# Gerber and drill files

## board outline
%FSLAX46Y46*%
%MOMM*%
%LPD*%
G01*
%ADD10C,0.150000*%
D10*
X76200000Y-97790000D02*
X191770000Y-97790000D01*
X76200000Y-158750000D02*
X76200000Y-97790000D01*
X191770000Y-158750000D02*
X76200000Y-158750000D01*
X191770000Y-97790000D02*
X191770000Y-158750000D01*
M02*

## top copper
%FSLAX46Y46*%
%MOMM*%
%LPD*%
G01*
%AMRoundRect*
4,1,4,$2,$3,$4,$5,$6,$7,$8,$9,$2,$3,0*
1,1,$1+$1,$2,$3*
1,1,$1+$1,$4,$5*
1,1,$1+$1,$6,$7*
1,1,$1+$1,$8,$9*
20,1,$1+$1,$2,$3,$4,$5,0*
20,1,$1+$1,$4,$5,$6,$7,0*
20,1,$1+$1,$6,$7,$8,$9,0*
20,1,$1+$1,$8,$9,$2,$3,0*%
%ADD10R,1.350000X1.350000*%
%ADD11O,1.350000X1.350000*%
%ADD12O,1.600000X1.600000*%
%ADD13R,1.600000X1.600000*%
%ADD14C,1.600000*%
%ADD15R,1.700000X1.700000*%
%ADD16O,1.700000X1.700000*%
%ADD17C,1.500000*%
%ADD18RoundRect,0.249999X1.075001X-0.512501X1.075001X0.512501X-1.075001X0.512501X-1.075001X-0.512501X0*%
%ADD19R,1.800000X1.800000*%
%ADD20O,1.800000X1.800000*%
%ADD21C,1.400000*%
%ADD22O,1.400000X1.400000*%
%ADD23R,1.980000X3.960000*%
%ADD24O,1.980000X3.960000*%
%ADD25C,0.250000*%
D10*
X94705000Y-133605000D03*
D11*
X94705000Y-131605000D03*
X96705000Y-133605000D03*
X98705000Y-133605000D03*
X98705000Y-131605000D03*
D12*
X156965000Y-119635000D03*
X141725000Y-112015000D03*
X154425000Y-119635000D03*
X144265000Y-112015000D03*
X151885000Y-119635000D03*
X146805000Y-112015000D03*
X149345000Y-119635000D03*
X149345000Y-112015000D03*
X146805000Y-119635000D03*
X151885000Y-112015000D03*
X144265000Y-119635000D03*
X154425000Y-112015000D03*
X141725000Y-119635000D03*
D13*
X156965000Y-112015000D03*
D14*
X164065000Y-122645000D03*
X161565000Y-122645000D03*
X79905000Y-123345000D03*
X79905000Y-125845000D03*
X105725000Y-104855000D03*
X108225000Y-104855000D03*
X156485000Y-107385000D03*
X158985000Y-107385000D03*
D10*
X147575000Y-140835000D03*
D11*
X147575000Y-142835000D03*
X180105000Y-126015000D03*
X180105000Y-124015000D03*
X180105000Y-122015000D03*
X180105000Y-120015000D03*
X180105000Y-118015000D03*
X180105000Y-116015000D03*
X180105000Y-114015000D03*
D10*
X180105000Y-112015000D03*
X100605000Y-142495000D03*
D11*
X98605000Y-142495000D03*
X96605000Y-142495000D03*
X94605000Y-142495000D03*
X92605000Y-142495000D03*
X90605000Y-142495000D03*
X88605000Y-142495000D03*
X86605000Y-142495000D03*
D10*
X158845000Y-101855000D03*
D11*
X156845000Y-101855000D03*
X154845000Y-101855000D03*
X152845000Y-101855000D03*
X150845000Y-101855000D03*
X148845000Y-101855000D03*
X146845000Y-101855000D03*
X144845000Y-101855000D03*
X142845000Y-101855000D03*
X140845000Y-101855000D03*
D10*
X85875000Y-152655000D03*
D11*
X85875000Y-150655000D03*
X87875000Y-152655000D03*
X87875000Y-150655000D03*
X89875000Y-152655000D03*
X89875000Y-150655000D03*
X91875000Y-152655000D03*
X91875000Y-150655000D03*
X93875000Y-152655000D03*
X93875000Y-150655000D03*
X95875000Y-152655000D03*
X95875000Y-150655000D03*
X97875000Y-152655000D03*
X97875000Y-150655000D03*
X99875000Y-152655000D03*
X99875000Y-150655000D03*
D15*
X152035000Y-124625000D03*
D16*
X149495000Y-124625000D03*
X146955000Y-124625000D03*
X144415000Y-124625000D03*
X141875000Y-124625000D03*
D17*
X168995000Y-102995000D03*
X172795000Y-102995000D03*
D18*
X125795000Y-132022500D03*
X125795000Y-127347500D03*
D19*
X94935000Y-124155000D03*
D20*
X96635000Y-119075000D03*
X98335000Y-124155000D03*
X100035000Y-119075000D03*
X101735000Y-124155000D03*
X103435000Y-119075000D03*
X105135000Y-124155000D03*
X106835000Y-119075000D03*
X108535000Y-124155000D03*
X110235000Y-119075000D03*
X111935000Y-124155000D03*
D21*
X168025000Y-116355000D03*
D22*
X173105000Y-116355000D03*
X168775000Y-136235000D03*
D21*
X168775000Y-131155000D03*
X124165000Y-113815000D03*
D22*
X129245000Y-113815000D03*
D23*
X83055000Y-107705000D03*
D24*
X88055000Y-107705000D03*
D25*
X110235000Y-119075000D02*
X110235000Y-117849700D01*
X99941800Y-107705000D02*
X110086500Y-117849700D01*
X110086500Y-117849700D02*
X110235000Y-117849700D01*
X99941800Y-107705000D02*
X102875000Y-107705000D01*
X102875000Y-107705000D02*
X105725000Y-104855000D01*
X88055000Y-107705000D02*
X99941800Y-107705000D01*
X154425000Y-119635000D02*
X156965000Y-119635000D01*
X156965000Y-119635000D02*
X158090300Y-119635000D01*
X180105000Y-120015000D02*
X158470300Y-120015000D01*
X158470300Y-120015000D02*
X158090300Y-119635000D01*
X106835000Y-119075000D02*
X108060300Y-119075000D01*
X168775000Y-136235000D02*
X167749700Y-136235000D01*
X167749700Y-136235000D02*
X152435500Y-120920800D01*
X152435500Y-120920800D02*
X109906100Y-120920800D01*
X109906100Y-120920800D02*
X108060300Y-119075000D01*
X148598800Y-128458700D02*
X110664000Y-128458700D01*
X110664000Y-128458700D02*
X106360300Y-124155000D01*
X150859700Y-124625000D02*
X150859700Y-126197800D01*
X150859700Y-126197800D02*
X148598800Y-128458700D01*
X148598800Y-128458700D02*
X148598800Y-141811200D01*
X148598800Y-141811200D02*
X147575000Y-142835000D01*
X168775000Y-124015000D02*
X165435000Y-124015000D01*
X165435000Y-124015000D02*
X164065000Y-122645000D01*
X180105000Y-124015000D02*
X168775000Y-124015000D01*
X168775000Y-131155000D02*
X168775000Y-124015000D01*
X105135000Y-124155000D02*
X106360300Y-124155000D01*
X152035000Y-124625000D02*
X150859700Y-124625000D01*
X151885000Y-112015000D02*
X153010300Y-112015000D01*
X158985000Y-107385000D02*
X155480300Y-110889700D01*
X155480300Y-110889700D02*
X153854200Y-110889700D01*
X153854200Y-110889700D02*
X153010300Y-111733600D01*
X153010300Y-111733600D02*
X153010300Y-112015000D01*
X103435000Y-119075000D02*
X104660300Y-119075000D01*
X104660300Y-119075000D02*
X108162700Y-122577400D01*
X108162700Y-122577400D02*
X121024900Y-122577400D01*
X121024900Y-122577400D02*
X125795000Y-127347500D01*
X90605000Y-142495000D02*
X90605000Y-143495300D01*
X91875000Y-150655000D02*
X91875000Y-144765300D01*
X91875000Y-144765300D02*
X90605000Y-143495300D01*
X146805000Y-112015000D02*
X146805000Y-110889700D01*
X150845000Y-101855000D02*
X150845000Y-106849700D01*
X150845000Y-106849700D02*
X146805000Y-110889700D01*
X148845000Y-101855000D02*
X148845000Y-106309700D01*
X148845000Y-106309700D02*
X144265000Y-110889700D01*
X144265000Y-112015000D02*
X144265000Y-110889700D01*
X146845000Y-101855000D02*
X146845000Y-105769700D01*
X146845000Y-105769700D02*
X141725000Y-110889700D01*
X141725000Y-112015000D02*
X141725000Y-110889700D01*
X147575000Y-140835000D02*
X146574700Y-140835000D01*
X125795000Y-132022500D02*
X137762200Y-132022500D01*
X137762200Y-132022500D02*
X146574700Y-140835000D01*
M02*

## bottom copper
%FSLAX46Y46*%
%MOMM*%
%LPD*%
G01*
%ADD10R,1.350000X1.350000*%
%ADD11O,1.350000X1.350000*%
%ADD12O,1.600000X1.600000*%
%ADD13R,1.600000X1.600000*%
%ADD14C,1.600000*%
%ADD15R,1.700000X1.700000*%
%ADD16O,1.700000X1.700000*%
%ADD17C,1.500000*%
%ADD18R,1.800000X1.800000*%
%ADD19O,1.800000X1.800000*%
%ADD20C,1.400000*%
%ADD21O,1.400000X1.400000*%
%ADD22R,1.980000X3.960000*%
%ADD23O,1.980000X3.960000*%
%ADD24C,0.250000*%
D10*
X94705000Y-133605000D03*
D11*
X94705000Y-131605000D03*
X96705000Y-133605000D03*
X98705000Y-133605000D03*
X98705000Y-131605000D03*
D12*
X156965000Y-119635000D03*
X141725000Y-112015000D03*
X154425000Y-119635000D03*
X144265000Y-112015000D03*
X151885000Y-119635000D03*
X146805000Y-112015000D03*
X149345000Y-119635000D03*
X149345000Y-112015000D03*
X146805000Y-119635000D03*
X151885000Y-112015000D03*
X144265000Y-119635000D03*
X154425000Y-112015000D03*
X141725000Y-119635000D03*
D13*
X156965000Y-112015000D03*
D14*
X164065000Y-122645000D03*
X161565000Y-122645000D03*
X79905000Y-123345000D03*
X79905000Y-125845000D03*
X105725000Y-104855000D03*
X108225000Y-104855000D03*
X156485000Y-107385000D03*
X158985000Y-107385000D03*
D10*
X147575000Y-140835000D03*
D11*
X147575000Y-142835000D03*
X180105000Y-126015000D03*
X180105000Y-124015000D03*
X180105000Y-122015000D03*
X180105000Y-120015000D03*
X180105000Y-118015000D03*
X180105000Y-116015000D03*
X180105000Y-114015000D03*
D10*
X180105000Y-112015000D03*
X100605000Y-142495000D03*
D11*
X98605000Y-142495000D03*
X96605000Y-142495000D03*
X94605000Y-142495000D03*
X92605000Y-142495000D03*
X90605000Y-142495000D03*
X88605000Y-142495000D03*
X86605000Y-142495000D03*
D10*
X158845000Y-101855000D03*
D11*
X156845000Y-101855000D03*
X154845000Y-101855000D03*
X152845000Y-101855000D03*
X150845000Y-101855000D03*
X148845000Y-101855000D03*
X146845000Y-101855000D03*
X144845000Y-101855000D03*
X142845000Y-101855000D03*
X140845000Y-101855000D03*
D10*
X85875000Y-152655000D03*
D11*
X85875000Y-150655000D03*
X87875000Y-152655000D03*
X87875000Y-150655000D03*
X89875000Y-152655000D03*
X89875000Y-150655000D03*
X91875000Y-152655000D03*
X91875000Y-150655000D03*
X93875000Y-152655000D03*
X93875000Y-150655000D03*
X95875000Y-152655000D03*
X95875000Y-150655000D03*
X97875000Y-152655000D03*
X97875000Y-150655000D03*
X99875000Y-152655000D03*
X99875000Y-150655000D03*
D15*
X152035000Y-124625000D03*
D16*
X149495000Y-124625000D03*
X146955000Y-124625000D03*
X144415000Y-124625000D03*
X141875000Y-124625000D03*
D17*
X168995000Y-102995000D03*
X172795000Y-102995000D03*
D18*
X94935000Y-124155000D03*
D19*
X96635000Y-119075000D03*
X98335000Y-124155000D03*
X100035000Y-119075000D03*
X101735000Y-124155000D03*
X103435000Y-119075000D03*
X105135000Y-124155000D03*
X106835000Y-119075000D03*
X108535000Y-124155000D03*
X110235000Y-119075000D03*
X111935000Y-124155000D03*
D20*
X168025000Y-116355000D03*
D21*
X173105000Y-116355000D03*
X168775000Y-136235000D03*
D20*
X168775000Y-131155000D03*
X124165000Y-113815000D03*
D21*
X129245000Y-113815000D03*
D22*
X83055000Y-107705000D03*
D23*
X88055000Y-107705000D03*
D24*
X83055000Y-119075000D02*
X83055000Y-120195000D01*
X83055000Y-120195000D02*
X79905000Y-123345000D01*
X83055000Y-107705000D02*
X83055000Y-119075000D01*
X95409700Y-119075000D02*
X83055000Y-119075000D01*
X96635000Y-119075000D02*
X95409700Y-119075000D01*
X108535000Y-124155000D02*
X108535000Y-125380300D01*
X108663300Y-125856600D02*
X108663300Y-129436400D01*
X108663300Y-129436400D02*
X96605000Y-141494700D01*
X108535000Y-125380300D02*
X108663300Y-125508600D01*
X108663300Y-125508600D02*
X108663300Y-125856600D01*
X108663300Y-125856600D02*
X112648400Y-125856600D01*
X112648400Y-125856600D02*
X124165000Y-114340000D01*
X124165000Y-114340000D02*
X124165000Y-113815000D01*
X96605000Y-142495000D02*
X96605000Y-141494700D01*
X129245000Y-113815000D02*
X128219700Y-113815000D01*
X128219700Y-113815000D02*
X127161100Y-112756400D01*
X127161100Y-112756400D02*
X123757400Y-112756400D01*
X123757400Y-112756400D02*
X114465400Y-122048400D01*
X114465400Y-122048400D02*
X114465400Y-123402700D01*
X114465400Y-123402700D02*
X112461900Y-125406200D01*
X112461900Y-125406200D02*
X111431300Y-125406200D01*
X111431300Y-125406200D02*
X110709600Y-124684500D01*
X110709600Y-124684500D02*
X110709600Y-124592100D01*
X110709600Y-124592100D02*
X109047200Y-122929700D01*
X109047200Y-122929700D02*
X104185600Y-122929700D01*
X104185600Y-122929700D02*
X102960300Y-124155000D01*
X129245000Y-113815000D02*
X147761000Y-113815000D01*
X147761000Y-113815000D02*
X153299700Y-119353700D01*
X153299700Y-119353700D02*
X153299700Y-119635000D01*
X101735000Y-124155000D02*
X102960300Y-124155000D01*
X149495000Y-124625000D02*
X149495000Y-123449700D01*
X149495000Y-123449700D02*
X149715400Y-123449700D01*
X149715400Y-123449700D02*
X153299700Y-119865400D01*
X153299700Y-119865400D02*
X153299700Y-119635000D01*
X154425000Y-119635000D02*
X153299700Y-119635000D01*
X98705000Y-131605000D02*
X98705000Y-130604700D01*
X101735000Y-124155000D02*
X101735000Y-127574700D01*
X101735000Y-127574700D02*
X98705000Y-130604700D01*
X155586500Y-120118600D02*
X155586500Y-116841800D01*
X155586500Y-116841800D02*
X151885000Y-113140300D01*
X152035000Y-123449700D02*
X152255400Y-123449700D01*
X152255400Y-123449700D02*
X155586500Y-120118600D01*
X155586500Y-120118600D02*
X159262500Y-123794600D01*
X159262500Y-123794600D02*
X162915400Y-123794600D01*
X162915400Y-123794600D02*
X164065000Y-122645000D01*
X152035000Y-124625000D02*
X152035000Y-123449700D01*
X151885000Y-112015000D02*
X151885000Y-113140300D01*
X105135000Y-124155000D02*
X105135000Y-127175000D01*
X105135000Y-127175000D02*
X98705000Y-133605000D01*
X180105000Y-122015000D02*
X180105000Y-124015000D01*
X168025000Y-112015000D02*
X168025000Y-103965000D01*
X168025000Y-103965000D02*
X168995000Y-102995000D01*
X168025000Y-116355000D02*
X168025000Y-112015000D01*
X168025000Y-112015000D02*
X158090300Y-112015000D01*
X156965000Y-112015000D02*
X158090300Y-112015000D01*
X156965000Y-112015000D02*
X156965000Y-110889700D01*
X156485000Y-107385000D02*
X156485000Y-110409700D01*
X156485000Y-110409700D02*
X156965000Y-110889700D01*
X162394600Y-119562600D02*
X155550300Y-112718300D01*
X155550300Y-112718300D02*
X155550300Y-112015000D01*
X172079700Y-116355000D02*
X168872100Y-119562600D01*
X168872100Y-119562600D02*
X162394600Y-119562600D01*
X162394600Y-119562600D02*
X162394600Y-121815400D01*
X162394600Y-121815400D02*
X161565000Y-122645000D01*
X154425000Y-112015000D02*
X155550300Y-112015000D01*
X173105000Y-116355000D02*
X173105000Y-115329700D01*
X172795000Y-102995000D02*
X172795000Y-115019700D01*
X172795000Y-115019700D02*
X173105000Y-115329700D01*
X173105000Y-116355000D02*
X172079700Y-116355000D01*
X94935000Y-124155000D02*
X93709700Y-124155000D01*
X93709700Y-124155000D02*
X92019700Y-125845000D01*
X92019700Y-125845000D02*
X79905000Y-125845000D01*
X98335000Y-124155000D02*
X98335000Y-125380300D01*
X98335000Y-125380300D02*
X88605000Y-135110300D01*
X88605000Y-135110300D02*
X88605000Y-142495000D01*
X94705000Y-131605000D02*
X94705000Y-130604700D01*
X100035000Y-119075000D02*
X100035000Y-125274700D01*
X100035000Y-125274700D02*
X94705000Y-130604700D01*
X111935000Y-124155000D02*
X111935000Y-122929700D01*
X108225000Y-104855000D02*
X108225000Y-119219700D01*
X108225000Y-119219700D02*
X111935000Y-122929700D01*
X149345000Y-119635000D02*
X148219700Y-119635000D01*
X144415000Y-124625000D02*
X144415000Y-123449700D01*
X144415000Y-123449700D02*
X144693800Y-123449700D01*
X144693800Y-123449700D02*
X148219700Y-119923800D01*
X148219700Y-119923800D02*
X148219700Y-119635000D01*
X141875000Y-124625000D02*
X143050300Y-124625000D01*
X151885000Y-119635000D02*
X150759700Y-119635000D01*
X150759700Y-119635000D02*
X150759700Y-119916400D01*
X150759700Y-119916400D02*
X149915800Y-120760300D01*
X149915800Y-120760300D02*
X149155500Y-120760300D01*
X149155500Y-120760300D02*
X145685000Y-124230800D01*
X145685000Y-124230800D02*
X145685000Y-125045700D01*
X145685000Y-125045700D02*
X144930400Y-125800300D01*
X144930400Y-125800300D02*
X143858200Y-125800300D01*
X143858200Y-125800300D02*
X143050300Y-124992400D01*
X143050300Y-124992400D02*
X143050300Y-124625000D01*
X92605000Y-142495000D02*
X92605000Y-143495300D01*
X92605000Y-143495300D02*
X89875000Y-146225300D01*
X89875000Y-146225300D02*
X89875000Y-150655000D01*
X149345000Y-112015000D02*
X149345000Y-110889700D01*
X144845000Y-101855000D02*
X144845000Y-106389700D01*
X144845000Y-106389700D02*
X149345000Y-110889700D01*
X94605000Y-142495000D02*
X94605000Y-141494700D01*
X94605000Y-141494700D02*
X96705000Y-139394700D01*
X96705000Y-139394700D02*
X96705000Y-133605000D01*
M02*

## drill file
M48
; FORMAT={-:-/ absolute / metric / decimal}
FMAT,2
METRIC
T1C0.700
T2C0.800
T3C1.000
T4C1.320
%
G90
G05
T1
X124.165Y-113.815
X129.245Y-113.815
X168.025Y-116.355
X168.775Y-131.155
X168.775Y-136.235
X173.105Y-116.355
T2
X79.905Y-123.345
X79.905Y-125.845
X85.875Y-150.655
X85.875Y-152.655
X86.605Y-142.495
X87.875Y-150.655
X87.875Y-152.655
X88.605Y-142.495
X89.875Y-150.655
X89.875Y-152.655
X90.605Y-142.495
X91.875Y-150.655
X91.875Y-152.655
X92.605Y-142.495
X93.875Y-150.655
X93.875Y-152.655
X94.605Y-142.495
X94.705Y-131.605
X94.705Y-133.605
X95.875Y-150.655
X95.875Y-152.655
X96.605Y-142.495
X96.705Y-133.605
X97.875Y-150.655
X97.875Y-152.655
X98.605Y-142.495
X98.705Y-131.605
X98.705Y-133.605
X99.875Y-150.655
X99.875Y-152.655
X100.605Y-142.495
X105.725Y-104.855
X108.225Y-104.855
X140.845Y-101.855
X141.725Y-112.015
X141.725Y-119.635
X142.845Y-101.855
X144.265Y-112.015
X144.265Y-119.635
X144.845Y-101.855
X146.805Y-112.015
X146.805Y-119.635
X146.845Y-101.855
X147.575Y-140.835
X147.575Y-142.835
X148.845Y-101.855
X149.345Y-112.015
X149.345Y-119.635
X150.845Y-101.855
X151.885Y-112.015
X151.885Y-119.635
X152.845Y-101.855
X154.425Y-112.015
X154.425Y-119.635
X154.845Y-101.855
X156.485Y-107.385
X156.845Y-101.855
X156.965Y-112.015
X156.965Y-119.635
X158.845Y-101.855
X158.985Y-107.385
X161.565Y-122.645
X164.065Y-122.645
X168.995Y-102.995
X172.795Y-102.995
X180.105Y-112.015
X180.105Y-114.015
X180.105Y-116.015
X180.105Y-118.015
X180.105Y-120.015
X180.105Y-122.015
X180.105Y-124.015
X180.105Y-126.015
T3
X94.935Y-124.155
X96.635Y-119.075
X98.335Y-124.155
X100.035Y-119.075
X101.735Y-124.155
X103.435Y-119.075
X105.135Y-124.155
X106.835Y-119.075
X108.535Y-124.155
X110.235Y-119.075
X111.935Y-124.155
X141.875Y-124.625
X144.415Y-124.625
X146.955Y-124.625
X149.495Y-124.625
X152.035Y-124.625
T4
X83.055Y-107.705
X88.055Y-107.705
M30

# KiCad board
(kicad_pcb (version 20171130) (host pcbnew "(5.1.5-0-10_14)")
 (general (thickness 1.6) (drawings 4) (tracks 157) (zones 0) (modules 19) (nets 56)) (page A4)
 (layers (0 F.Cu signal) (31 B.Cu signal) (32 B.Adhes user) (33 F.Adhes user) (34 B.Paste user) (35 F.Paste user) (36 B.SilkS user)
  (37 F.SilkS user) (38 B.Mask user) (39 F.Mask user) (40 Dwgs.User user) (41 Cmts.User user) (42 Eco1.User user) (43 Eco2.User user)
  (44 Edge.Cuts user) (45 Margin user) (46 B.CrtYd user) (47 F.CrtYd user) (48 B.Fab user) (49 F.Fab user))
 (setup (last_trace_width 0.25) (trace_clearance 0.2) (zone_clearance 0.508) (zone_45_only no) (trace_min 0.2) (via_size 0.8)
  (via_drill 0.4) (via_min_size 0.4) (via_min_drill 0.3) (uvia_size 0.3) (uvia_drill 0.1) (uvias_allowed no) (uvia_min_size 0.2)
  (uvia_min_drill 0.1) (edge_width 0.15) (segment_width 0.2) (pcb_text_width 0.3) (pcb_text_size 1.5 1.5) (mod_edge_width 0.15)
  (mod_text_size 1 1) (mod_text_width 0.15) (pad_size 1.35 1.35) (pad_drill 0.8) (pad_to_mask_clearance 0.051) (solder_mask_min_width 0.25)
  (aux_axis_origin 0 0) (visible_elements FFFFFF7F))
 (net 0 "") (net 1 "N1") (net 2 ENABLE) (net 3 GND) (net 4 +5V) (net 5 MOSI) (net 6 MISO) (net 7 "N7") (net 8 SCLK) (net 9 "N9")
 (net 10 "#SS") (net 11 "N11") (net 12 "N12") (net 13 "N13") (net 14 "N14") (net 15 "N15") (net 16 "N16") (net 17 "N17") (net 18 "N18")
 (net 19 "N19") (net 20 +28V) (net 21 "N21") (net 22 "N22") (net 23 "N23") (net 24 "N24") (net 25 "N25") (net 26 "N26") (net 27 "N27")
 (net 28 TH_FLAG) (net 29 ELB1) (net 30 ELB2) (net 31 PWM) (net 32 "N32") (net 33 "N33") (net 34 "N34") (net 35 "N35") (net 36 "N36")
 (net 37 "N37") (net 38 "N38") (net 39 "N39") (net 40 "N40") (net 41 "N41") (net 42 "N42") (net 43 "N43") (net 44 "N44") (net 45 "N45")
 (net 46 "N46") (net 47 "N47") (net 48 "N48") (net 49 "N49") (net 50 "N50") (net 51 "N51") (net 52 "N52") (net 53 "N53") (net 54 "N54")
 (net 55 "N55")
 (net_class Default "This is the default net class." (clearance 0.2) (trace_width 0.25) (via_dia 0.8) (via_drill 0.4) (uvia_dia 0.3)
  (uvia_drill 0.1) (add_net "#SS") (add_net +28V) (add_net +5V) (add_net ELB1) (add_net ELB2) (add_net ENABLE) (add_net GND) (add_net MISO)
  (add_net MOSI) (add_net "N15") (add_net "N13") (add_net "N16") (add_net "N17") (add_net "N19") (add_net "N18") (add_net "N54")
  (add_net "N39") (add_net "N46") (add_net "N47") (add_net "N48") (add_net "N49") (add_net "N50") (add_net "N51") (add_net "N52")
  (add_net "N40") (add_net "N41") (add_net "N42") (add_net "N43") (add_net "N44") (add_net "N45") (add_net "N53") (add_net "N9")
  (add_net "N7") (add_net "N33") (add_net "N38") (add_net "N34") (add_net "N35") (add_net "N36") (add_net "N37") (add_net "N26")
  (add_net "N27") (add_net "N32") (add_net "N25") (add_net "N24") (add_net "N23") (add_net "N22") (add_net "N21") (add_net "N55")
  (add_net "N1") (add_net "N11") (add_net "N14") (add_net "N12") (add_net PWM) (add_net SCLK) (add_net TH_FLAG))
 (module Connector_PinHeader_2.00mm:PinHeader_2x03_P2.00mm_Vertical (layer F.Cu) (at 94.705 133.605 90)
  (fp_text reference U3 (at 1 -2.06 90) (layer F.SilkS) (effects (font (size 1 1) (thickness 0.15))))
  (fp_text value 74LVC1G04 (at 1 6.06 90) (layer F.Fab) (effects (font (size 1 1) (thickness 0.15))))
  (pad 1 thru_hole rect (at 0 0 90) (size 1.35 1.35) (drill 0.8) (layers *.Cu *.Mask))
  (pad 4 thru_hole oval (at 2 0 90) (size 1.35 1.35) (drill 0.8) (layers *.Cu *.Mask) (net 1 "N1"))
  (pad 2 thru_hole oval (at 0 2 90) (size 1.35 1.35) (drill 0.8) (layers *.Cu *.Mask) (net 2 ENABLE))
  (pad 3 thru_hole oval (at 0 4 90) (size 1.35 1.35) (drill 0.8) (layers *.Cu *.Mask) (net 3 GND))
  (pad 5 thru_hole oval (at 2 4 90) (size 1.35 1.35) (drill 0.8) (layers *.Cu *.Mask) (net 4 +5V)))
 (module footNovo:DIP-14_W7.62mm (layer F.Cu) (at 156.965 112.015 270)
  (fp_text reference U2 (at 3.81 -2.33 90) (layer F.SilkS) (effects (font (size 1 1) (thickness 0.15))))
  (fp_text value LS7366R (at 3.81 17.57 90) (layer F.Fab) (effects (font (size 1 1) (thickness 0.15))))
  (pad 14 thru_hole oval (at 7.62 0 270) (size 1.6 1.6) (drill 0.8) (layers *.Cu *.Mask) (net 4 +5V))
  (pad 7 thru_hole oval (at 0 15.24 270) (size 1.6 1.6) (drill 0.8) (layers *.Cu *.Mask) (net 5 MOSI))
  (pad 13 thru_hole oval (at 7.62 2.54 270) (size 1.6 1.6) (drill 0.8) (layers *.Cu *.Mask) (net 4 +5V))
  (pad 6 thru_hole oval (at 0 12.7 270) (size 1.6 1.6) (drill 0.8) (layers *.Cu *.Mask) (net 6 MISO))
  (pad 12 thru_hole oval (at 7.62 5.08 270) (size 1.6 1.6) (drill 0.8) (layers *.Cu *.Mask) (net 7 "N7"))
  (pad 5 thru_hole oval (at 0 10.16 270) (size 1.6 1.6) (drill 0.8) (layers *.Cu *.Mask) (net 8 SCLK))
  (pad 11 thru_hole oval (at 7.62 7.62 270) (size 1.6 1.6) (drill 0.8) (layers *.Cu *.Mask) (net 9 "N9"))
  (pad 4 thru_hole oval (at 0 7.62 270) (size 1.6 1.6) (drill 0.8) (layers *.Cu *.Mask) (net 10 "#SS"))
  (pad 10 thru_hole oval (at 7.62 10.16 270) (size 1.6 1.6) (drill 0.8) (layers *.Cu *.Mask) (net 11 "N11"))
  (pad 3 thru_hole oval (at 0 5.08 270) (size 1.6 1.6) (drill 0.8) (layers *.Cu *.Mask) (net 3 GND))
  (pad 9 thru_hole oval (at 7.62 12.7 270) (size 1.6 1.6) (drill 0.8) (layers *.Cu *.Mask) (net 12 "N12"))
  (pad 2 thru_hole oval (at 0 2.54 270) (size 1.6 1.6) (drill 0.8) (layers *.Cu *.Mask) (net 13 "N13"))
  (pad 8 thru_hole oval (at 7.62 15.24 270) (size 1.6 1.6) (drill 0.8) (layers *.Cu *.Mask) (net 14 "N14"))
  (pad 1 thru_hole rect (at 0 0 270) (size 1.6 1.6) (drill 0.8) (layers *.Cu *.Mask) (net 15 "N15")))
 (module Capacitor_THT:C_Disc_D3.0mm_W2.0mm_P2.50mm (layer F.Cu) (at 161.565 122.645)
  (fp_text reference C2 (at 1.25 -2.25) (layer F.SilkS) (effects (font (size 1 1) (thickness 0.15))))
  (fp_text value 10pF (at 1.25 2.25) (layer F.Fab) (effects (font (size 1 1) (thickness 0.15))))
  (pad 2 thru_hole circle (at 2.5 0) (size 1.6 1.6) (drill 0.8) (layers *.Cu *.Mask) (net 3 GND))
  (pad 1 thru_hole circle (at 0 0) (size 1.6 1.6) (drill 0.8) (layers *.Cu *.Mask) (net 13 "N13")))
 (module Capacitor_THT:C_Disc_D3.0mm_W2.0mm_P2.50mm (layer F.Cu) (at 79.905 123.345 270)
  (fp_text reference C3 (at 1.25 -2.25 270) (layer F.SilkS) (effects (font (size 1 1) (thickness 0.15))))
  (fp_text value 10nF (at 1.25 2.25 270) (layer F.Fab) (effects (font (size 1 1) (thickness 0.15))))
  (pad 1 thru_hole circle (at 0 0 270) (size 1.6 1.6) (drill 0.8) (layers *.Cu *.Mask) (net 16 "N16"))
  (pad 2 thru_hole circle (at 2.5 0 270) (size 1.6 1.6) (drill 0.8) (layers *.Cu *.Mask) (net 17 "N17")))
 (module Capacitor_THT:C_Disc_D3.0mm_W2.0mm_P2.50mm (layer F.Cu) (at 108.225 104.855 180)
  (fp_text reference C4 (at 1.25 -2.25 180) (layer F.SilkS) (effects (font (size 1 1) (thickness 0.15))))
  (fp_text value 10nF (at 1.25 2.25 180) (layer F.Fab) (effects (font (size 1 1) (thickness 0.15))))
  (pad 2 thru_hole circle (at 2.5 0 180) (size 1.6 1.6) (drill 0.8) (layers *.Cu *.Mask) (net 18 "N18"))
  (pad 1 thru_hole circle (at 0 0 180) (size 1.6 1.6) (drill 0.8) (layers *.Cu *.Mask) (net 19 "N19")))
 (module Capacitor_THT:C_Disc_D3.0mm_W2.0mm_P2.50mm (layer F.Cu) (at 156.485 107.385)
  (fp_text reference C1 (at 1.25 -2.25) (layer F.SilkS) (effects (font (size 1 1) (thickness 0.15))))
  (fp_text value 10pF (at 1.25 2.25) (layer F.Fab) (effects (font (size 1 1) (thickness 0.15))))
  (pad 1 thru_hole circle (at 0 0) (size 1.6 1.6) (drill 0.8) (layers *.Cu *.Mask) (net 15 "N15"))
  (pad 2 thru_hole circle (at 2.5 0) (size 1.6 1.6) (drill 0.8) (layers *.Cu *.Mask) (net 3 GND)))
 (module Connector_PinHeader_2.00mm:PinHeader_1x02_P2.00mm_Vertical (layer F.Cu) (at 147.575 140.835)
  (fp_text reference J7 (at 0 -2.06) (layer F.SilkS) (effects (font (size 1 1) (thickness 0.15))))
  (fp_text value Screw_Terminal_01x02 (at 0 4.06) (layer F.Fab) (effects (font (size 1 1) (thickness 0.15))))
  (pad 1 thru_hole rect (at 0 0) (size 1.35 1.35) (drill 0.8) (layers *.Cu *.Mask) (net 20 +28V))
  (pad 2 thru_hole oval (at 0 2) (size 1.35 1.35) (drill 0.8) (layers *.Cu *.Mask) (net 3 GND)))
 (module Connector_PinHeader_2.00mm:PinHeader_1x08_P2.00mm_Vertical (layer F.Cu) (at 180.105 112.015)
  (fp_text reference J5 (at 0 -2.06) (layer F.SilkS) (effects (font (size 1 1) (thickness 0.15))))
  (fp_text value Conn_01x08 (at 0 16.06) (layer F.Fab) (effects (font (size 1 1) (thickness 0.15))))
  (pad 8 thru_hole oval (at 0 14) (size 1.35 1.35) (drill 0.8) (layers *.Cu *.Mask) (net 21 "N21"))
  (pad 7 thru_hole oval (at 0 12) (size 1.35 1.35) (drill 0.8) (layers *.Cu *.Mask) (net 3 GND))
  (pad 6 thru_hole oval (at 0 10) (size 1.35 1.35) (drill 0.8) (layers *.Cu *.Mask) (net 3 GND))
  (pad 5 thru_hole oval (at 0 8) (size 1.35 1.35) (drill 0.8) (layers *.Cu *.Mask) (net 4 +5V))
  (pad 4 thru_hole oval (at 0 6) (size 1.35 1.35) (drill 0.8) (layers *.Cu *.Mask) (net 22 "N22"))
  (pad 3 thru_hole oval (at 0 4) (size 1.35 1.35) (drill 0.8) (layers *.Cu *.Mask) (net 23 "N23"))
  (pad 2 thru_hole oval (at 0 2) (size 1.35 1.35) (drill 0.8) (layers *.Cu *.Mask) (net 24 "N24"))
  (pad 1 thru_hole rect (at 0 0) (size 1.35 1.35) (drill 0.8) (layers *.Cu *.Mask) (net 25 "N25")))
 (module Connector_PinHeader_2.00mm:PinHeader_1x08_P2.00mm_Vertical (layer F.Cu) (at 100.605 142.495 270)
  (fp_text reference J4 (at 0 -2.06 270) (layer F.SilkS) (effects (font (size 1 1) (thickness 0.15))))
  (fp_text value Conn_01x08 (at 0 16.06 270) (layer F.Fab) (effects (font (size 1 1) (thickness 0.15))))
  (pad 1 thru_hole rect (at 0 0 270) (size 1.35 1.35) (drill 0.8) (layers *.Cu *.Mask) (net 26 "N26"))
  (pad 2 thru_hole oval (at 0 2 270) (size 1.35 1.35) (drill 0.8) (layers *.Cu *.Mask) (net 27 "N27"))
  (pad 3 thru_hole oval (at 0 4 270) (size 1.35 1.35) (drill 0.8) (layers *.Cu *.Mask) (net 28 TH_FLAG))
  (pad 4 thru_hole oval (at 0 6 270) (size 1.35 1.35) (drill 0.8) (layers *.Cu *.Mask) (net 2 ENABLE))
  (pad 5 thru_hole oval (at 0 8 270) (size 1.35 1.35) (drill 0.8) (layers *.Cu *.Mask) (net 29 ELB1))
  (pad 6 thru_hole oval (at 0 10 270) (size 1.35 1.35) (drill 0.8) (layers *.Cu *.Mask) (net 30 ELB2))
  (pad 7 thru_hole oval (at 0 12 270) (size 1.35 1.35) (drill 0.8) (layers *.Cu *.Mask) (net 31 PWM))
  (pad 8 thru_hole oval (at 0 14 270) (size 1.35 1.35) (drill 0.8) (layers *.Cu *.Mask) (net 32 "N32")))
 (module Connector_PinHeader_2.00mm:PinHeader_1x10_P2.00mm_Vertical (layer F.Cu) (at 158.845 101.855 270)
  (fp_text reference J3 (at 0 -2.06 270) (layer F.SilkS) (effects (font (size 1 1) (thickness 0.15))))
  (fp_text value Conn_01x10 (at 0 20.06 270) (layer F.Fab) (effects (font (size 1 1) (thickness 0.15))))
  (pad 1 thru_hole rect (at 0 0 270) (size 1.35 1.35) (drill 0.8) (layers *.Cu *.Mask) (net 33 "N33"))
  (pad 2 thru_hole oval (at 0 2 270) (size 1.35 1.35) (drill 0.8) (layers *.Cu *.Mask) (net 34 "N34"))
  (pad 3 thru_hole oval (at 0 4 270) (size 1.35 1.35) (drill 0.8) (layers *.Cu *.Mask) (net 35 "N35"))
  (pad 4 thru_hole oval (at 0 6 270) (size 1.35 1.35) (drill 0.8) (layers *.Cu *.Mask) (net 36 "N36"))
  (pad 5 thru_hole oval (at 0 8 270) (size 1.35 1.35) (drill 0.8) (layers *.Cu *.Mask) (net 8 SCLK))
  (pad 6 thru_hole oval (at 0 10 270) (size 1.35 1.35) (drill 0.8) (layers *.Cu *.Mask) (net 6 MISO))
  (pad 7 thru_hole oval (at 0 12 270) (size 1.35 1.35) (drill 0.8) (layers *.Cu *.Mask) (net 5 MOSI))
  (pad 8 thru_hole oval (at 0 14 270) (size 1.35 1.35) (drill 0.8) (layers *.Cu *.Mask) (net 10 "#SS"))
  (pad 9 thru_hole oval (at 0 16 270) (size 1.35 1.35) (drill 0.8) (layers *.Cu *.Mask) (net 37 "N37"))
  (pad 10 thru_hole oval (at 0 18 270) (size 1.35 1.35) (drill 0.8) (layers *.Cu *.Mask) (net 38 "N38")))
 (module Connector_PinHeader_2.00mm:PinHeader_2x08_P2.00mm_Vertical (layer F.Cu) (at 85.875 152.655 90)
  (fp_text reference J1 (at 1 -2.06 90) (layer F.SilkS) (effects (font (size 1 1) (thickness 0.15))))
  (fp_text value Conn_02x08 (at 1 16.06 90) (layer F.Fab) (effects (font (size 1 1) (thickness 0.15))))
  (pad 1 thru_hole rect (at 0 0 90) (size 1.35 1.35) (drill 0.8) (layers *.Cu *.Mask) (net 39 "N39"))
  (pad 2 thru_hole oval (at 2 0 90) (size 1.35 1.35) (drill 0.8) (layers *.Cu *.Mask) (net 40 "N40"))
  (pad 3 thru_hole oval (at 0 2 90) (size 1.35 1.35) (drill 0.8) (layers *.Cu *.Mask) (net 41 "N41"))
  (pad 4 thru_hole oval (at 2 2 90) (size 1.35 1.35) (drill 0.8) (layers *.Cu *.Mask) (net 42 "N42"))
  (pad 5 thru_hole oval (at 0 4 90) (size 1.35 1.35) (drill 0.8) (layers *.Cu *.Mask) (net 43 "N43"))
  (pad 6 thru_hole oval (at 2 4 90) (size 1.35 1.35) (drill 0.8) (layers *.Cu *.Mask) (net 29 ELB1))
  (pad 7 thru_hole oval (at 0 6 90) (size 1.35 1.35) (drill 0.8) (layers *.Cu *.Mask) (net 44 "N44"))
  (pad 8 thru_hole oval (at 2 6 90) (size 1.35 1.35) (drill 0.8) (layers *.Cu *.Mask) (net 30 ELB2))
  (pad 9 thru_hole oval (at 0 8 90) (size 1.35 1.35) (drill 0.8) (layers *.Cu *.Mask) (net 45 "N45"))
  (pad 10 thru_hole oval (at 2 8 90) (size 1.35 1.35) (drill 0.8) (layers *.Cu *.Mask) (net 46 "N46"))
  (pad 11 thru_hole oval (at 0 10 90) (size 1.35 1.35) (drill 0.8) (layers *.Cu *.Mask) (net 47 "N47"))
  (pad 12 thru_hole oval (at 2 10 90) (size 1.35 1.35) (drill 0.8) (layers *.Cu *.Mask) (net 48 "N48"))
  (pad 13 thru_hole oval (at 0 12 90) (size 1.35 1.35) (drill 0.8) (layers *.Cu *.Mask) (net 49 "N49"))
  (pad 14 thru_hole oval (at 2 12 90) (size 1.35 1.35) (drill 0.8) (layers *.Cu *.Mask) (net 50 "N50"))
  (pad 15 thru_hole oval (at 0 14 90) (size 1.35 1.35) (drill 0.8) (layers *.Cu *.Mask) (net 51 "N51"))
  (pad 16 thru_hole oval (at 2 14 90) (size 1.35 1.35) (drill 0.8) (layers *.Cu *.Mask) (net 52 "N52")))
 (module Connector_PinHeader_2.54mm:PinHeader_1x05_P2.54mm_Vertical (layer F.Cu) (at 152.035 124.625 270)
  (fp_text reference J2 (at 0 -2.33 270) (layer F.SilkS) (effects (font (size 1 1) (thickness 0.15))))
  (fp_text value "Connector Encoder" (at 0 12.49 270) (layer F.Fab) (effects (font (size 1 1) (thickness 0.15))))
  (pad 1 thru_hole rect (at 0 0 270) (size 1.7 1.7) (drill 1) (layers *.Cu *.Mask) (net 3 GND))
  (pad 2 thru_hole oval (at 0 2.54 270) (size 1.7 1.7) (drill 1) (layers *.Cu *.Mask) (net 4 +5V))
  (pad 3 thru_hole oval (at 0 5.08 270) (size 1.7 1.7) (drill 1) (layers *.Cu *.Mask) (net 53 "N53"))
  (pad 4 thru_hole oval (at 0 7.62 270) (size 1.7 1.7) (drill 1) (layers *.Cu *.Mask) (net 9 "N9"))
  (pad 5 thru_hole oval (at 0 10.16 270) (size 1.7 1.7) (drill 1) (layers *.Cu *.Mask) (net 7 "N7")))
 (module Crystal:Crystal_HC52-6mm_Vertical (layer F.Cu) (at 168.995 102.995)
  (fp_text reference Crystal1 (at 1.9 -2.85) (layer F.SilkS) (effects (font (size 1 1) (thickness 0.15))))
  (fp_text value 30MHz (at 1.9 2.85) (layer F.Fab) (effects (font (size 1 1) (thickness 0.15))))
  (pad 1 thru_hole circle (at 0 0) (size 1.5 1.5) (drill 0.8) (layers *.Cu *.Mask) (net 15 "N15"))
  (pad 2 thru_hole circle (at 3.8 0) (size 1.5 1.5) (drill 0.8) (layers *.Cu *.Mask) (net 13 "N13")))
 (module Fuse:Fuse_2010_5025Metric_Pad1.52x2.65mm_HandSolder (layer F.Cu) (at 125.795 129.685 90)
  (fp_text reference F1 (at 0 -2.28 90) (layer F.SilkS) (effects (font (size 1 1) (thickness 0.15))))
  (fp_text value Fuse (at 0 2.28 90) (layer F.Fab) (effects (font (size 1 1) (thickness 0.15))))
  (pad 1 smd roundrect (at -2.3375 0 90) (size 1.525 2.65) (layers F.Cu F.Paste F.Mask) (roundrect_rratio 0.163934) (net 20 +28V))
  (pad 2 smd roundrect (at 2.3375 0 90) (size 1.525 2.65) (layers F.Cu F.Paste F.Mask) (roundrect_rratio 0.163934) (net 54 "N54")))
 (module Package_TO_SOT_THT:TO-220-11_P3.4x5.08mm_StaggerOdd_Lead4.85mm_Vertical (layer F.Cu) (at 94.935 124.155)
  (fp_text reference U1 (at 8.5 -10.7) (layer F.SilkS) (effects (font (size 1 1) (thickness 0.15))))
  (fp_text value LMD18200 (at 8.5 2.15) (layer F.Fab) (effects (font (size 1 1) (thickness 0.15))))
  (pad 1 thru_hole rect (at 0 0) (size 1.8 1.8) (drill 1) (layers *.Cu *.Mask) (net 17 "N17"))
  (pad 2 thru_hole oval (at 1.7 -5.08) (size 1.8 1.8) (drill 1) (layers *.Cu *.Mask) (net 16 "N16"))
  (pad 3 thru_hole oval (at 3.4 0) (size 1.8 1.8) (drill 1) (layers *.Cu *.Mask) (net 31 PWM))
  (pad 4 thru_hole oval (at 5.1 -5.08) (size 1.8 1.8) (drill 1) (layers *.Cu *.Mask) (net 1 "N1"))
  (pad 5 thru_hole oval (at 6.8 0) (size 1.8 1.8) (drill 1) (layers *.Cu *.Mask) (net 4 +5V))
  (pad 6 thru_hole oval (at 8.5 -5.08) (size 1.8 1.8) (drill 1) (layers *.Cu *.Mask) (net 54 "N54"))
  (pad 7 thru_hole oval (at 10.2 0) (size 1.8 1.8) (drill 1) (layers *.Cu *.Mask) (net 3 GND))
  (pad 8 thru_hole oval (at 11.9 -5.08) (size 1.8 1.8) (drill 1) (layers *.Cu *.Mask) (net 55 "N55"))
  (pad 9 thru_hole oval (at 13.6 0) (size 1.8 1.8) (drill 1) (layers *.Cu *.Mask) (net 28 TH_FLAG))
  (pad 10 thru_hole oval (at 15.3 -5.08) (size 1.8 1.8) (drill 1) (layers *.Cu *.Mask) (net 18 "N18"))
  (pad 11 thru_hole oval (at 17 0) (size 1.8 1.8) (drill 1) (layers *.Cu *.Mask) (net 19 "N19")))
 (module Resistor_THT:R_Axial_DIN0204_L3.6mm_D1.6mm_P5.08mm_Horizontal (layer F.Cu) (at 168.025 116.355)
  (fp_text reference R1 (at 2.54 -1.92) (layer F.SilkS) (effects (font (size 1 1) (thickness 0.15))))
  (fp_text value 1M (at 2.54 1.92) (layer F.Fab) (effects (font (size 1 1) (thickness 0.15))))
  (pad 1 thru_hole circle (at 0 0) (size 1.4 1.4) (drill 0.7) (layers *.Cu *.Mask) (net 15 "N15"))
  (pad 2 thru_hole oval (at 5.08 0) (size 1.4 1.4) (drill 0.7) (layers *.Cu *.Mask) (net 13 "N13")))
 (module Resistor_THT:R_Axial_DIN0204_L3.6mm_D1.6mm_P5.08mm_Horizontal (layer F.Cu) (at 168.775 131.155 270)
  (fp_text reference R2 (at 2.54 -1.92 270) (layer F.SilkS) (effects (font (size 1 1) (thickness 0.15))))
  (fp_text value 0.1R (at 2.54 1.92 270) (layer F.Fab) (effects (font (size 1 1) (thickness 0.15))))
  (pad 2 thru_hole oval (at 5.08 0 270) (size 1.4 1.4) (drill 0.7) (layers *.Cu *.Mask) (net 55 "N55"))
  (pad 1 thru_hole circle (at 0 0 270) (size 1.4 1.4) (drill 0.7) (layers *.Cu *.Mask) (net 3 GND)))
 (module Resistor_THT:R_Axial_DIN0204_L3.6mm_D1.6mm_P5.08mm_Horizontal (layer F.Cu) (at 124.165 113.815)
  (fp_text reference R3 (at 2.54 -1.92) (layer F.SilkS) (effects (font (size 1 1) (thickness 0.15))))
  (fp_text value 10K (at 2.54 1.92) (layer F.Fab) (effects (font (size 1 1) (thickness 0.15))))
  (pad 1 thru_hole circle (at 0 0) (size 1.4 1.4) (drill 0.7) (layers *.Cu *.Mask) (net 28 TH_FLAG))
  (pad 2 thru_hole oval (at 5.08 0) (size 1.4 1.4) (drill 0.7) (layers *.Cu *.Mask) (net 4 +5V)))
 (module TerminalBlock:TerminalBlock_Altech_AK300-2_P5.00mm (layer F.Cu) (at 83.055 107.705)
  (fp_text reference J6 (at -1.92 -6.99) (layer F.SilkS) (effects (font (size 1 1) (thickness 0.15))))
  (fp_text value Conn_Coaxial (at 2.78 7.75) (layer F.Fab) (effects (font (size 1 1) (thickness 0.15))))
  (pad 1 thru_hole rect (at 0 0) (size 1.98 3.96) (drill 1.32) (layers *.Cu *.Mask) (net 16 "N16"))
  (pad 2 thru_hole oval (at 5 0) (size 1.98 3.96) (drill 1.32) (layers *.Cu *.Mask) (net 18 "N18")))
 (gr_line (start 76.2 97.79) (end 191.77 97.79) (angle 90) (layer Edge.Cuts) (width 0.15))
 (gr_line (start 76.2 158.75) (end 76.2 97.79) (angle 90) (layer Edge.Cuts) (width 0.15))
 (gr_line (start 191.77 158.75) (end 76.2 158.75) (angle 90) (layer Edge.Cuts) (width 0.15))
 (gr_line (start 191.77 97.79) (end 191.77 158.75) (angle 90) (layer Edge.Cuts) (width 0.15))
 (segment (start 83.055 119.075) (end 83.055 120.195) (width 0.25) (layer B.Cu) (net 16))
 (segment (start 83.055 120.195) (end 79.905 123.345) (width 0.25) (layer B.Cu) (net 16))
 (segment (start 83.055 107.705) (end 83.055 119.075) (width 0.25) (layer B.Cu) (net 16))
 (segment (start 95.4097 119.075) (end 83.055 119.075) (width 0.25) (layer B.Cu) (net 16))
 (segment (start 96.635 119.075) (end 95.4097 119.075) (width 0.25) (layer B.Cu) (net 16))
 (segment (start 110.235 119.075) (end 110.235 117.8497) (width 0.25) (layer F.Cu) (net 18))
 (segment (start 99.9418 107.705) (end 110.0865 117.8497) (width 0.25) (layer F.Cu) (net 18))
 (segment (start 110.0865 117.8497) (end 110.235 117.8497) (width 0.25) (layer F.Cu) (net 18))
 (segment (start 99.9418 107.705) (end 102.875 107.705) (width 0.25) (layer F.Cu) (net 18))
 (segment (start 102.875 107.705) (end 105.725 104.855) (width 0.25) (layer F.Cu) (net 18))
 (segment (start 88.055 107.705) (end 99.9418 107.705) (width 0.25) (layer F.Cu) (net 18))
 (segment (start 108.535 124.155) (end 108.535 125.3803) (width 0.25) (layer B.Cu) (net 28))
 (segment (start 108.6633 125.8566) (end 108.6633 129.4364) (width 0.25) (layer B.Cu) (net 28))
 (segment (start 108.6633 129.4364) (end 96.605 141.4947) (width 0.25) (layer B.Cu) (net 28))
 (segment (start 108.535 125.3803) (end 108.6633 125.5086) (width 0.25) (layer B.Cu) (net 28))
 (segment (start 108.6633 125.5086) (end 108.6633 125.8566) (width 0.25) (layer B.Cu) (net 28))
 (segment (start 108.6633 125.8566) (end 112.6484 125.8566) (width 0.25) (layer B.Cu) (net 28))
 (segment (start 112.6484 125.8566) (end 124.165 114.34) (width 0.25) (layer B.Cu) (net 28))
 (segment (start 124.165 114.34) (end 124.165 113.815) (width 0.25) (layer B.Cu) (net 28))
 (segment (start 96.605 142.495) (end 96.605 141.4947) (width 0.25) (layer B.Cu) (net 28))
 (segment (start 129.245 113.815) (end 128.2197 113.815) (width 0.25) (layer B.Cu) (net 4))
 (segment (start 128.2197 113.815) (end 127.1611 112.7564) (width 0.25) (layer B.Cu) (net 4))
 (segment (start 127.1611 112.7564) (end 123.7574 112.7564) (width 0.25) (layer B.Cu) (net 4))
 (segment (start 123.7574 112.7564) (end 114.4654 122.0484) (width 0.25) (layer B.Cu) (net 4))
 (segment (start 114.4654 122.0484) (end 114.4654 123.4027) (width 0.25) (layer B.Cu) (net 4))
 (segment (start 114.4654 123.4027) (end 112.4619 125.4062) (width 0.25) (layer B.Cu) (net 4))
 (segment (start 112.4619 125.4062) (end 111.4313 125.4062) (width 0.25) (layer B.Cu) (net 4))
 (segment (start 111.4313 125.4062) (end 110.7096 124.6845) (width 0.25) (layer B.Cu) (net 4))
 (segment (start 110.7096 124.6845) (end 110.7096 124.5921) (width 0.25) (layer B.Cu) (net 4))
 (segment (start 110.7096 124.5921) (end 109.0472 122.9297) (width 0.25) (layer B.Cu) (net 4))
 (segment (start 109.0472 122.9297) (end 104.1856 122.9297) (width 0.25) (layer B.Cu) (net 4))
 (segment (start 104.1856 122.9297) (end 102.9603 124.155) (width 0.25) (layer B.Cu) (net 4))
 (segment (start 129.245 113.815) (end 147.761 113.815) (width 0.25) (layer B.Cu) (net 4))
 (segment (start 147.761 113.815) (end 153.2997 119.3537) (width 0.25) (layer B.Cu) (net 4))
 (segment (start 153.2997 119.3537) (end 153.2997 119.635) (width 0.25) (layer B.Cu) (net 4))
 (segment (start 101.735 124.155) (end 102.9603 124.155) (width 0.25) (layer B.Cu) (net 4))
 (segment (start 149.495 124.625) (end 149.495 123.4497) (width 0.25) (layer B.Cu) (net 4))
 (segment (start 149.495 123.4497) (end 149.7154 123.4497) (width 0.25) (layer B.Cu) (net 4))
 (segment (start 149.7154 123.4497) (end 153.2997 119.8654) (width 0.25) (layer B.Cu) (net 4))
 (segment (start 153.2997 119.8654) (end 153.2997 119.635) (width 0.25) (layer B.Cu) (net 4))
 (segment (start 154.425 119.635) (end 153.2997 119.635) (width 0.25) (layer B.Cu) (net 4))
 (segment (start 154.425 119.635) (end 156.965 119.635) (width 0.25) (layer F.Cu) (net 4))
 (segment (start 156.965 119.635) (end 158.0903 119.635) (width 0.25) (layer F.Cu) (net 4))
 (segment (start 180.105 120.015) (end 158.4703 120.015) (width 0.25) (layer F.Cu) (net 4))
 (segment (start 158.4703 120.015) (end 158.0903 119.635) (width 0.25) (layer F.Cu) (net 4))
 (segment (start 98.705 131.605) (end 98.705 130.6047) (width 0.25) (layer B.Cu) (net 4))
 (segment (start 101.735 124.155) (end 101.735 127.5747) (width 0.25) (layer B.Cu) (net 4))
 (segment (start 101.735 127.5747) (end 98.705 130.6047) (width 0.25) (layer B.Cu) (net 4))
 (segment (start 106.835 119.075) (end 108.0603 119.075) (width 0.25) (layer F.Cu) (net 55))
 (segment (start 168.775 136.235) (end 167.7497 136.235) (width 0.25) (layer F.Cu) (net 55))
 (segment (start 167.7497 136.235) (end 152.4355 120.9208) (width 0.25) (layer F.Cu) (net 55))
 (segment (start 152.4355 120.9208) (end 109.9061 120.9208) (width 0.25) (layer F.Cu) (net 55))
 (segment (start 109.9061 120.9208) (end 108.0603 119.075) (width 0.25) (layer F.Cu) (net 55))
 (segment (start 148.5988 128.4587) (end 110.664 128.4587) (width 0.25) (layer F.Cu) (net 3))
 (segment (start 110.664 128.4587) (end 106.3603 124.155) (width 0.25) (layer F.Cu) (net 3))
 (segment (start 150.8597 124.625) (end 150.8597 126.1978) (width 0.25) (layer F.Cu) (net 3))
 (segment (start 150.8597 126.1978) (end 148.5988 128.4587) (width 0.25) (layer F.Cu) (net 3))
 (segment (start 148.5988 128.4587) (end 148.5988 141.8112) (width 0.25) (layer F.Cu) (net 3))
 (segment (start 148.5988 141.8112) (end 147.575 142.835) (width 0.25) (layer F.Cu) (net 3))
 (segment (start 155.5865 120.1186) (end 155.5865 116.8418) (width 0.25) (layer B.Cu) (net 3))
 (segment (start 155.5865 116.8418) (end 151.885 113.1403) (width 0.25) (layer B.Cu) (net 3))
 (segment (start 152.035 123.4497) (end 152.2554 123.4497) (width 0.25) (layer B.Cu) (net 3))
 (segment (start 152.2554 123.4497) (end 155.5865 120.1186) (width 0.25) (layer B.Cu) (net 3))
 (segment (start 155.5865 120.1186) (end 159.2625 123.7946) (width 0.25) (layer B.Cu) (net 3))
 (segment (start 159.2625 123.7946) (end 162.9154 123.7946) (width 0.25) (layer B.Cu) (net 3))
 (segment (start 162.9154 123.7946) (end 164.065 122.645) (width 0.25) (layer B.Cu) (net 3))
 (segment (start 152.035 124.625) (end 152.035 123.4497) (width 0.25) (layer B.Cu) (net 3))
 (segment (start 151.885 112.015) (end 151.885 113.1403) (width 0.25) (layer B.Cu) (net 3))
 (segment (start 168.775 124.015) (end 165.435 124.015) (width 0.25) (layer F.Cu) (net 3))
 (segment (start 165.435 124.015) (end 164.065 122.645) (width 0.25) (layer F.Cu) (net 3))
 (segment (start 180.105 124.015) (end 168.775 124.015) (width 0.25) (layer F.Cu) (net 3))
 (segment (start 168.775 131.155) (end 168.775 124.015) (width 0.25) (layer F.Cu) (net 3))
 (segment (start 105.135 124.155) (end 105.135 127.175) (width 0.25) (layer B.Cu) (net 3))
 (segment (start 105.135 127.175) (end 98.705 133.605) (width 0.25) (layer B.Cu) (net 3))
 (segment (start 105.135 124.155) (end 106.3603 124.155) (width 0.25) (layer F.Cu) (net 3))
 (segment (start 152.035 124.625) (end 150.8597 124.625) (width 0.25) (layer F.Cu) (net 3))
 (segment (start 151.885 112.015) (end 153.0103 112.015) (width 0.25) (layer F.Cu) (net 3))
 (segment (start 158.985 107.385) (end 155.4803 110.8897) (width 0.25) (layer F.Cu) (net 3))
 (segment (start 155.4803 110.8897) (end 153.8542 110.8897) (width 0.25) (layer F.Cu) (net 3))
 (segment (start 153.8542 110.8897) (end 153.0103 111.7336) (width 0.25) (layer F.Cu) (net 3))
 (segment (start 153.0103 111.7336) (end 153.0103 112.015) (width 0.25) (layer F.Cu) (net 3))
 (segment (start 180.105 122.015) (end 180.105 124.015) (width 0.25) (layer B.Cu) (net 3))
 (segment (start 168.025 112.015) (end 168.025 103.965) (width 0.25) (layer B.Cu) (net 15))
 (segment (start 168.025 103.965) (end 168.995 102.995) (width 0.25) (layer B.Cu) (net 15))
 (segment (start 168.025 116.355) (end 168.025 112.015) (width 0.25) (layer B.Cu) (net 15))
 (segment (start 168.025 112.015) (end 158.0903 112.015) (width 0.25) (layer B.Cu) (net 15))
 (segment (start 156.965 112.015) (end 158.0903 112.015) (width 0.25) (layer B.Cu) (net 15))
 (segment (start 156.965 112.015) (end 156.965 110.8897) (width 0.25) (layer B.Cu) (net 15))
 (segment (start 156.485 107.385) (end 156.485 110.4097) (width 0.25) (layer B.Cu) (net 15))
 (segment (start 156.485 110.4097) (end 156.965 110.8897) (width 0.25) (layer B.Cu) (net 15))
 (segment (start 162.3946 119.5626) (end 155.5503 112.7183) (width 0.25) (layer B.Cu) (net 13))
 (segment (start 155.5503 112.7183) (end 155.5503 112.015) (width 0.25) (layer B.Cu) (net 13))
 (segment (start 172.0797 116.355) (end 168.8721 119.5626) (width 0.25) (layer B.Cu) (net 13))
 (segment (start 168.8721 119.5626) (end 162.3946 119.5626) (width 0.25) (layer B.Cu) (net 13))
 (segment (start 162.3946 119.5626) (end 162.3946 121.8154) (width 0.25) (layer B.Cu) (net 13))
 (segment (start 162.3946 121.8154) (end 161.565 122.645) (width 0.25) (layer B.Cu) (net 13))
 (segment (start 154.425 112.015) (end 155.5503 112.015) (width 0.25) (layer B.Cu) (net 13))
 (segment (start 173.105 116.355) (end 173.105 115.3297) (width 0.25) (layer B.Cu) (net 13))
 (segment (start 172.795 102.995) (end 172.795 115.0197) (width 0.25) (layer B.Cu) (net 13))
 (segment (start 172.795 115.0197) (end 173.105 115.3297) (width 0.25) (layer B.Cu) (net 13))
 (segment (start 173.105 116.355) (end 172.0797 116.355) (width 0.25) (layer B.Cu) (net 13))
 (segment (start 94.935 124.155) (end 93.7097 124.155) (width 0.25) (layer B.Cu) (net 17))
 (segment (start 93.7097 124.155) (end 92.0197 125.845) (width 0.25) (layer B.Cu) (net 17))
 (segment (start 92.0197 125.845) (end 79.905 125.845) (width 0.25) (layer B.Cu) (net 17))
 (segment (start 98.335 124.155) (end 98.335 125.3803) (width 0.25) (layer B.Cu) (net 31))
 (segment (start 98.335 125.3803) (end 88.605 135.1103) (width 0.25) (layer B.Cu) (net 31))
 (segment (start 88.605 135.1103) (end 88.605 142.495) (width 0.25) (layer B.Cu) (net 31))
 (segment (start 94.705 131.605) (end 94.705 130.6047) (width 0.25) (layer B.Cu) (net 1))
 (segment (start 100.035 119.075) (end 100.035 125.2747) (width 0.25) (layer B.Cu) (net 1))
 (segment (start 100.035 125.2747) (end 94.705 130.6047) (width 0.25) (layer B.Cu) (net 1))
 (segment (start 103.435 119.075) (end 104.6603 119.075) (width 0.25) (layer F.Cu) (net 54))
 (segment (start 104.6603 119.075) (end 108.1627 122.5774) (width 0.25) (layer F.Cu) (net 54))
 (segment (start 108.1627 122.5774) (end 121.0249 122.5774) (width 0.25) (layer F.Cu) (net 54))
 (segment (start 121.0249 122.5774) (end 125.795 127.3475) (width 0.25) (layer F.Cu) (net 54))
 (segment (start 111.935 124.155) (end 111.935 122.9297) (width 0.25) (layer B.Cu) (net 19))
 (segment (start 108.225 104.855) (end 108.225 119.2197) (width 0.25) (layer B.Cu) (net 19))
 (segment (start 108.225 119.2197) (end 111.935 122.9297) (width 0.25) (layer B.Cu) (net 19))
 (segment (start 149.345 119.635) (end 148.2197 119.635) (width 0.25) (layer B.Cu) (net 9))
 (segment (start 144.415 124.625) (end 144.415 123.4497) (width 0.25) (layer B.Cu) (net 9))
 (segment (start 144.415 123.4497) (end 144.6938 123.4497) (width 0.25) (layer B.Cu) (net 9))
 (segment (start 144.6938 123.4497) (end 148.2197 119.9238) (width 0.25) (layer B.Cu) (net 9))
 (segment (start 148.2197 119.9238) (end 148.2197 119.635) (width 0.25) (layer B.Cu) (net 9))
 (segment (start 141.875 124.625) (end 143.0503 124.625) (width 0.25) (layer B.Cu) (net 7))
 (segment (start 151.885 119.635) (end 150.7597 119.635) (width 0.25) (layer B.Cu) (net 7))
 (segment (start 150.7597 119.635) (end 150.7597 119.9164) (width 0.25) (layer B.Cu) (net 7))
 (segment (start 150.7597 119.9164) (end 149.9158 120.7603) (width 0.25) (layer B.Cu) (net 7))
 (segment (start 149.9158 120.7603) (end 149.1555 120.7603) (width 0.25) (layer B.Cu) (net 7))
 (segment (start 149.1555 120.7603) (end 145.685 124.2308) (width 0.25) (layer B.Cu) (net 7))
 (segment (start 145.685 124.2308) (end 145.685 125.0457) (width 0.25) (layer B.Cu) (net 7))
 (segment (start 145.685 125.0457) (end 144.9304 125.8003) (width 0.25) (layer B.Cu) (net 7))
 (segment (start 144.9304 125.8003) (end 143.8582 125.8003) (width 0.25) (layer B.Cu) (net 7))
 (segment (start 143.8582 125.8003) (end 143.0503 124.9924) (width 0.25) (layer B.Cu) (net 7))
 (segment (start 143.0503 124.9924) (end 143.0503 124.625) (width 0.25) (layer B.Cu) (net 7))
 (segment (start 92.605 142.495) (end 92.605 143.4953) (width 0.25) (layer B.Cu) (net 29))
 (segment (start 92.605 143.4953) (end 89.875 146.2253) (width 0.25) (layer B.Cu) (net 29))
 (segment (start 89.875 146.2253) (end 89.875 150.655) (width 0.25) (layer B.Cu) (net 29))
 (segment (start 90.605 142.495) (end 90.605 143.4953) (width 0.25) (layer F.Cu) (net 30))
 (segment (start 91.875 150.655) (end 91.875 144.7653) (width 0.25) (layer F.Cu) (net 30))
 (segment (start 91.875 144.7653) (end 90.605 143.4953) (width 0.25) (layer F.Cu) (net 30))
 (segment (start 149.345 112.015) (end 149.345 110.8897) (width 0.25) (layer B.Cu) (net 10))
 (segment (start 144.845 101.855) (end 144.845 106.3897) (width 0.25) (layer B.Cu) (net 10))
 (segment (start 144.845 106.3897) (end 149.345 110.8897) (width 0.25) (layer B.Cu) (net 10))
 (segment (start 146.805 112.015) (end 146.805 110.8897) (width 0.25) (layer F.Cu) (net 8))
 (segment (start 150.845 101.855) (end 150.845 106.8497) (width 0.25) (layer F.Cu) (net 8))
 (segment (start 150.845 106.8497) (end 146.805 110.8897) (width 0.25) (layer F.Cu) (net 8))
 (segment (start 148.845 101.855) (end 148.845 106.3097) (width 0.25) (layer F.Cu) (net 6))
 (segment (start 148.845 106.3097) (end 144.265 110.8897) (width 0.25) (layer F.Cu) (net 6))
 (segment (start 144.265 112.015) (end 144.265 110.8897) (width 0.25) (layer F.Cu) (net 6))
 (segment (start 146.845 101.855) (end 146.845 105.7697) (width 0.25) (layer F.Cu) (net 5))
 (segment (start 146.845 105.7697) (end 141.725 110.8897) (width 0.25) (layer F.Cu) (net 5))
 (segment (start 141.725 112.015) (end 141.725 110.8897) (width 0.25) (layer F.Cu) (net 5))
 (segment (start 94.605 142.495) (end 94.605 141.4947) (width 0.25) (layer B.Cu) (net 2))
 (segment (start 94.605 141.4947) (end 96.705 139.3947) (width 0.25) (layer B.Cu) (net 2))
 (segment (start 96.705 139.3947) (end 96.705 133.605) (width 0.25) (layer B.Cu) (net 2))
 (segment (start 147.575 140.835) (end 146.5747 140.835) (width 0.25) (layer F.Cu) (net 20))
 (segment (start 125.795 132.0225) (end 137.7622 132.0225) (width 0.25) (layer F.Cu) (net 20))
 (segment (start 137.7622 132.0225) (end 146.5747 140.835) (width 0.25) (layer F.Cu) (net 20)))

